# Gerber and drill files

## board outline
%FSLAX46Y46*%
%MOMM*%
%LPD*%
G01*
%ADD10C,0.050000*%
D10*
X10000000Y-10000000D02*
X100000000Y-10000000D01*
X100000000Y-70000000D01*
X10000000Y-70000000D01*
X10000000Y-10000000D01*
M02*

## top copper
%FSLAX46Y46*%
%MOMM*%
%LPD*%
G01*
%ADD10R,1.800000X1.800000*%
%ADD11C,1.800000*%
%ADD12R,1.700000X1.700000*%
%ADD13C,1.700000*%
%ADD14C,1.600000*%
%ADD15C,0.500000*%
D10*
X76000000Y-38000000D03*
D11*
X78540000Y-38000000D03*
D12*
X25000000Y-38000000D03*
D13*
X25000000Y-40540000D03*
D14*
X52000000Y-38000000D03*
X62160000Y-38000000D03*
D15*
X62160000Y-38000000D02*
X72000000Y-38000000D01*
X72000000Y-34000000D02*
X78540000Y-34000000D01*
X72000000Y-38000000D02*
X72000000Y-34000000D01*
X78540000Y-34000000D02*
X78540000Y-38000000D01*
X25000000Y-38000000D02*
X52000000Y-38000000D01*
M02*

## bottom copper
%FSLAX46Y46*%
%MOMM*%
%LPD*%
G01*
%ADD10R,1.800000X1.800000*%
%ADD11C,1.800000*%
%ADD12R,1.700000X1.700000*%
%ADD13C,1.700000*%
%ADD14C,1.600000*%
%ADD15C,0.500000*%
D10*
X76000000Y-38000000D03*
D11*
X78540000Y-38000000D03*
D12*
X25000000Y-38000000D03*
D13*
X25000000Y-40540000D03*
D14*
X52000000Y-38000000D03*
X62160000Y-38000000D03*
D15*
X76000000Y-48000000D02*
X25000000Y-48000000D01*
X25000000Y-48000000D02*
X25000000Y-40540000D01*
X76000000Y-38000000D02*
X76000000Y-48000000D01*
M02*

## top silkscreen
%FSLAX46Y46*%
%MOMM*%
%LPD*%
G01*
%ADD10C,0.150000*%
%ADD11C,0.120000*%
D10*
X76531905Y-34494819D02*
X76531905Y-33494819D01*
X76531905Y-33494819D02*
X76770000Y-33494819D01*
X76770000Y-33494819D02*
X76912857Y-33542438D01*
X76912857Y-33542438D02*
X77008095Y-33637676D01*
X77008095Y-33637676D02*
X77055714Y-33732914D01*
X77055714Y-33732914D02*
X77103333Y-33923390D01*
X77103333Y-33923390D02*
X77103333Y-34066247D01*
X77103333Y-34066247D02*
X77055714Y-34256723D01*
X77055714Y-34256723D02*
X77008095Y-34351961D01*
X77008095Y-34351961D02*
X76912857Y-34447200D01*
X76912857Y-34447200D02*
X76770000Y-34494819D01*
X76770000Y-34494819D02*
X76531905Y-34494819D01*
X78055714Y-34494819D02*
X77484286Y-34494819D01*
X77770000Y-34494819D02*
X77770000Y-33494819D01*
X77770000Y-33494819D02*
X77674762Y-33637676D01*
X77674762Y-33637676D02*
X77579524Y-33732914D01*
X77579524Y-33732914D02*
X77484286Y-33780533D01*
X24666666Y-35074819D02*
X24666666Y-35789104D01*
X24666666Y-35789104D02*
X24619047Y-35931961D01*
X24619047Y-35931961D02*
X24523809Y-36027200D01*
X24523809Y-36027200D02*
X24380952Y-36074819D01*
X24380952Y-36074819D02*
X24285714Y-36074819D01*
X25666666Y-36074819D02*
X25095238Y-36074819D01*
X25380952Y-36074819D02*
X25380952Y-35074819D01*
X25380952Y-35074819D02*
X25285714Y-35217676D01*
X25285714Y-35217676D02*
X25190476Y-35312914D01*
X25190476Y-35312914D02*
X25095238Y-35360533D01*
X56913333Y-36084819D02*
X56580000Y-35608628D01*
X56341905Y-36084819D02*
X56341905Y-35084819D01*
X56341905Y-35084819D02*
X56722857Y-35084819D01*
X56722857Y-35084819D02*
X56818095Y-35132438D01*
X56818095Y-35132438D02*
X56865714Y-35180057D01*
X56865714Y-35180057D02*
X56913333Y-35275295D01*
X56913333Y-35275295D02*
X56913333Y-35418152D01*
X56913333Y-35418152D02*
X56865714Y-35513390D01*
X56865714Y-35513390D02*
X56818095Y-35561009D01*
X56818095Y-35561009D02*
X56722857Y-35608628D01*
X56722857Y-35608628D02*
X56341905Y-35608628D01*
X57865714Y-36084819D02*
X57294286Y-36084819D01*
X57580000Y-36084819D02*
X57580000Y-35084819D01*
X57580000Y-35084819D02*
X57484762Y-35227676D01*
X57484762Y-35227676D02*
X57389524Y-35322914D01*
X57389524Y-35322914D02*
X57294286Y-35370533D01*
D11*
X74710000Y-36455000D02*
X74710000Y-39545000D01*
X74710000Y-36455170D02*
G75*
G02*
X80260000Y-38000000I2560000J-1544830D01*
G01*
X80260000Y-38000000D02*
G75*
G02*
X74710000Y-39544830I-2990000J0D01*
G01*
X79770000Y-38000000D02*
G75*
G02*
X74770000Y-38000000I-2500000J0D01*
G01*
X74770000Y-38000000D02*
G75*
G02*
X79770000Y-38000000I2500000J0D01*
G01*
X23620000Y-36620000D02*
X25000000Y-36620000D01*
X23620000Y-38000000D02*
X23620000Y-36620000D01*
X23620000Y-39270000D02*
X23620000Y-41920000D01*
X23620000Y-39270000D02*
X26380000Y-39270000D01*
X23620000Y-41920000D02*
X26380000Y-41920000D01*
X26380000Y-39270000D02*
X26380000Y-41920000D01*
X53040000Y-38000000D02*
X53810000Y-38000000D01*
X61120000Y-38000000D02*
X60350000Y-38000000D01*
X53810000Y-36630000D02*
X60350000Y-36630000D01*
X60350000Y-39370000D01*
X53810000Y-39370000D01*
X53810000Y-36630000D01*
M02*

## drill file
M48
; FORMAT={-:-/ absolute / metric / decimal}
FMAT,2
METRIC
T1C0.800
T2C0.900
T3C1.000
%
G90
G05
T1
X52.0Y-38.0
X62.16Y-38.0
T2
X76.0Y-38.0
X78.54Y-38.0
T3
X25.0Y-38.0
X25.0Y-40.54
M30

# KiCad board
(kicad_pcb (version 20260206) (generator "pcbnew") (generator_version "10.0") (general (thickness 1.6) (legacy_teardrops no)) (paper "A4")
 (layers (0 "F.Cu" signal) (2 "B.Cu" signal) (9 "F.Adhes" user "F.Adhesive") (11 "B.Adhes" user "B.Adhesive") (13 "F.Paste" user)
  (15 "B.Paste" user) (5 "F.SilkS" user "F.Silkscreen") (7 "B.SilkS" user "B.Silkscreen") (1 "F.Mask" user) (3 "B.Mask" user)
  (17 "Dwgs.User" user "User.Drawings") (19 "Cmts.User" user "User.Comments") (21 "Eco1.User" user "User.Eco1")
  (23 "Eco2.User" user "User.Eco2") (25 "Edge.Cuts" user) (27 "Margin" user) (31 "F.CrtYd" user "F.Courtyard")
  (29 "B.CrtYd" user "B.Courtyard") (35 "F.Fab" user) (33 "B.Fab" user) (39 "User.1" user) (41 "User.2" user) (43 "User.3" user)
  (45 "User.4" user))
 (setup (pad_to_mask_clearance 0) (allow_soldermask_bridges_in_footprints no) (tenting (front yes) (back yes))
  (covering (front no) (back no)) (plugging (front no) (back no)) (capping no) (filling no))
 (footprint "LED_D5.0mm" (layer "F.Cu") (at 76 38)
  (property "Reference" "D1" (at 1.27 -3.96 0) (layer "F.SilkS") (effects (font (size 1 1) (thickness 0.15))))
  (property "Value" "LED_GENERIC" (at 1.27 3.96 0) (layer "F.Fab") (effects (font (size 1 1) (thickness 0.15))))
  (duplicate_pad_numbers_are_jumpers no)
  (fp_line (start -1.29 -1.545) (end -1.29 1.545) (stroke (width 0.12) (type solid)) (layer "F.SilkS"))
  (fp_arc (start -1.29 -1.54483) (mid 2.071779 -2.880495) (end 4.26 0) (stroke (width 0.12) (type solid)) (layer "F.SilkS"))
  (fp_arc (start 4.26 0) (mid 2.071779 2.880495) (end -1.29 1.54483) (stroke (width 0.12) (type solid)) (layer "F.SilkS"))
  (fp_circle (center 1.27 0) (end 3.77 0) (stroke (width 0.12) (type solid)) (fill no) (layer "F.SilkS"))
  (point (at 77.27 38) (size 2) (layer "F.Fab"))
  (pad "1" thru_hole rect (at 0 0) (size 1.8 1.8) (drill 0.9) (layers "*.Cu" "*.Mask") (remove_unused_layers no) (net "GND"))
  (pad "2" thru_hole circle (at 2.54 0) (size 1.8 1.8) (drill 0.9) (layers "*.Cu" "*.Mask") (remove_unused_layers no) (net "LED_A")))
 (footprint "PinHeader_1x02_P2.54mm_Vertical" (layer "F.Cu") (at 25 38)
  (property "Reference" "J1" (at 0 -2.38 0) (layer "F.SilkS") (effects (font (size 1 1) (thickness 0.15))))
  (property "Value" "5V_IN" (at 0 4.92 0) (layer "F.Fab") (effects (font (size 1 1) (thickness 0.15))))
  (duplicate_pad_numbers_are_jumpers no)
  (fp_line (start -1.38 -1.38) (end 0 -1.38) (stroke (width 0.12) (type solid)) (layer "F.SilkS"))
  (fp_line (start -1.38 0) (end -1.38 -1.38) (stroke (width 0.12) (type solid)) (layer "F.SilkS"))
  (fp_line (start -1.38 1.27) (end -1.38 3.92) (stroke (width 0.12) (type solid)) (layer "F.SilkS"))
  (fp_line (start -1.38 1.27) (end 1.38 1.27) (stroke (width 0.12) (type solid)) (layer "F.SilkS"))
  (fp_line (start -1.38 3.92) (end 1.38 3.92) (stroke (width 0.12) (type solid)) (layer "F.SilkS"))
  (fp_line (start 1.38 1.27) (end 1.38 3.92) (stroke (width 0.12) (type solid)) (layer "F.SilkS"))
  (pad "1" thru_hole rect (at 0 0) (size 1.7 1.7) (drill 1) (layers "*.Cu" "*.Mask") (remove_unused_layers no) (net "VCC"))
  (pad "2" thru_hole circle (at 0 2.54) (size 1.7 1.7) (drill 1) (layers "*.Cu" "*.Mask") (remove_unused_layers no) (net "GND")))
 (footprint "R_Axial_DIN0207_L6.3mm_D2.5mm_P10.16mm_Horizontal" (layer "F.Cu") (at 52 38)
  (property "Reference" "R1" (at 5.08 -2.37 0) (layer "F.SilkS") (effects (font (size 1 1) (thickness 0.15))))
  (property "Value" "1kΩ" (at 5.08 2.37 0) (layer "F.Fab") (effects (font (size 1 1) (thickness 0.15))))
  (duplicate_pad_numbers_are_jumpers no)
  (fp_line (start 1.04 0) (end 1.81 0) (stroke (width 0.12) (type solid)) (layer "F.SilkS"))
  (fp_line (start 9.12 0) (end 8.35 0) (stroke (width 0.12) (type solid)) (layer "F.SilkS"))
  (fp_rect (start 1.81 -1.37) (end 8.35 1.37) (stroke (width 0.12) (type solid)) (fill no) (layer "F.SilkS"))
  (pad "1" thru_hole circle (at 0 0) (size 1.6 1.6) (drill 0.8) (layers "*.Cu" "*.Mask") (remove_unused_layers no) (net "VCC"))
  (pad "2" thru_hole circle (at 10.16 0) (size 1.6 1.6) (drill 0.8) (layers "*.Cu" "*.Mask") (remove_unused_layers no) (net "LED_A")))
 (gr_rect (start 10 10) (end 100 70) (stroke (width 0.05) (type default)) (fill no) (layer "Edge.Cuts"))
 (segment (start 76 48) (end 25 48) (width 0.5) (layer "B.Cu") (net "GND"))
 (segment (start 25 48) (end 25 40.54) (width 0.5) (layer "B.Cu") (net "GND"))
 (segment (start 76 38) (end 76 48) (width 0.5) (layer "B.Cu") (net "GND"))
 (segment (start 62.16 38) (end 72 38) (width 0.5) (layer "F.Cu") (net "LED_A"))
 (segment (start 72 34) (end 78.54 34) (width 0.5) (layer "F.Cu") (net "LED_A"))
 (segment (start 72 38) (end 72 34) (width 0.5) (layer "F.Cu") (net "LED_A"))
 (segment (start 78.54 34) (end 78.54 38) (width 0.5) (layer "F.Cu") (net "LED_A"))
 (segment (start 25 38) (end 52 38) (width 0.5) (layer "F.Cu") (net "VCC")))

